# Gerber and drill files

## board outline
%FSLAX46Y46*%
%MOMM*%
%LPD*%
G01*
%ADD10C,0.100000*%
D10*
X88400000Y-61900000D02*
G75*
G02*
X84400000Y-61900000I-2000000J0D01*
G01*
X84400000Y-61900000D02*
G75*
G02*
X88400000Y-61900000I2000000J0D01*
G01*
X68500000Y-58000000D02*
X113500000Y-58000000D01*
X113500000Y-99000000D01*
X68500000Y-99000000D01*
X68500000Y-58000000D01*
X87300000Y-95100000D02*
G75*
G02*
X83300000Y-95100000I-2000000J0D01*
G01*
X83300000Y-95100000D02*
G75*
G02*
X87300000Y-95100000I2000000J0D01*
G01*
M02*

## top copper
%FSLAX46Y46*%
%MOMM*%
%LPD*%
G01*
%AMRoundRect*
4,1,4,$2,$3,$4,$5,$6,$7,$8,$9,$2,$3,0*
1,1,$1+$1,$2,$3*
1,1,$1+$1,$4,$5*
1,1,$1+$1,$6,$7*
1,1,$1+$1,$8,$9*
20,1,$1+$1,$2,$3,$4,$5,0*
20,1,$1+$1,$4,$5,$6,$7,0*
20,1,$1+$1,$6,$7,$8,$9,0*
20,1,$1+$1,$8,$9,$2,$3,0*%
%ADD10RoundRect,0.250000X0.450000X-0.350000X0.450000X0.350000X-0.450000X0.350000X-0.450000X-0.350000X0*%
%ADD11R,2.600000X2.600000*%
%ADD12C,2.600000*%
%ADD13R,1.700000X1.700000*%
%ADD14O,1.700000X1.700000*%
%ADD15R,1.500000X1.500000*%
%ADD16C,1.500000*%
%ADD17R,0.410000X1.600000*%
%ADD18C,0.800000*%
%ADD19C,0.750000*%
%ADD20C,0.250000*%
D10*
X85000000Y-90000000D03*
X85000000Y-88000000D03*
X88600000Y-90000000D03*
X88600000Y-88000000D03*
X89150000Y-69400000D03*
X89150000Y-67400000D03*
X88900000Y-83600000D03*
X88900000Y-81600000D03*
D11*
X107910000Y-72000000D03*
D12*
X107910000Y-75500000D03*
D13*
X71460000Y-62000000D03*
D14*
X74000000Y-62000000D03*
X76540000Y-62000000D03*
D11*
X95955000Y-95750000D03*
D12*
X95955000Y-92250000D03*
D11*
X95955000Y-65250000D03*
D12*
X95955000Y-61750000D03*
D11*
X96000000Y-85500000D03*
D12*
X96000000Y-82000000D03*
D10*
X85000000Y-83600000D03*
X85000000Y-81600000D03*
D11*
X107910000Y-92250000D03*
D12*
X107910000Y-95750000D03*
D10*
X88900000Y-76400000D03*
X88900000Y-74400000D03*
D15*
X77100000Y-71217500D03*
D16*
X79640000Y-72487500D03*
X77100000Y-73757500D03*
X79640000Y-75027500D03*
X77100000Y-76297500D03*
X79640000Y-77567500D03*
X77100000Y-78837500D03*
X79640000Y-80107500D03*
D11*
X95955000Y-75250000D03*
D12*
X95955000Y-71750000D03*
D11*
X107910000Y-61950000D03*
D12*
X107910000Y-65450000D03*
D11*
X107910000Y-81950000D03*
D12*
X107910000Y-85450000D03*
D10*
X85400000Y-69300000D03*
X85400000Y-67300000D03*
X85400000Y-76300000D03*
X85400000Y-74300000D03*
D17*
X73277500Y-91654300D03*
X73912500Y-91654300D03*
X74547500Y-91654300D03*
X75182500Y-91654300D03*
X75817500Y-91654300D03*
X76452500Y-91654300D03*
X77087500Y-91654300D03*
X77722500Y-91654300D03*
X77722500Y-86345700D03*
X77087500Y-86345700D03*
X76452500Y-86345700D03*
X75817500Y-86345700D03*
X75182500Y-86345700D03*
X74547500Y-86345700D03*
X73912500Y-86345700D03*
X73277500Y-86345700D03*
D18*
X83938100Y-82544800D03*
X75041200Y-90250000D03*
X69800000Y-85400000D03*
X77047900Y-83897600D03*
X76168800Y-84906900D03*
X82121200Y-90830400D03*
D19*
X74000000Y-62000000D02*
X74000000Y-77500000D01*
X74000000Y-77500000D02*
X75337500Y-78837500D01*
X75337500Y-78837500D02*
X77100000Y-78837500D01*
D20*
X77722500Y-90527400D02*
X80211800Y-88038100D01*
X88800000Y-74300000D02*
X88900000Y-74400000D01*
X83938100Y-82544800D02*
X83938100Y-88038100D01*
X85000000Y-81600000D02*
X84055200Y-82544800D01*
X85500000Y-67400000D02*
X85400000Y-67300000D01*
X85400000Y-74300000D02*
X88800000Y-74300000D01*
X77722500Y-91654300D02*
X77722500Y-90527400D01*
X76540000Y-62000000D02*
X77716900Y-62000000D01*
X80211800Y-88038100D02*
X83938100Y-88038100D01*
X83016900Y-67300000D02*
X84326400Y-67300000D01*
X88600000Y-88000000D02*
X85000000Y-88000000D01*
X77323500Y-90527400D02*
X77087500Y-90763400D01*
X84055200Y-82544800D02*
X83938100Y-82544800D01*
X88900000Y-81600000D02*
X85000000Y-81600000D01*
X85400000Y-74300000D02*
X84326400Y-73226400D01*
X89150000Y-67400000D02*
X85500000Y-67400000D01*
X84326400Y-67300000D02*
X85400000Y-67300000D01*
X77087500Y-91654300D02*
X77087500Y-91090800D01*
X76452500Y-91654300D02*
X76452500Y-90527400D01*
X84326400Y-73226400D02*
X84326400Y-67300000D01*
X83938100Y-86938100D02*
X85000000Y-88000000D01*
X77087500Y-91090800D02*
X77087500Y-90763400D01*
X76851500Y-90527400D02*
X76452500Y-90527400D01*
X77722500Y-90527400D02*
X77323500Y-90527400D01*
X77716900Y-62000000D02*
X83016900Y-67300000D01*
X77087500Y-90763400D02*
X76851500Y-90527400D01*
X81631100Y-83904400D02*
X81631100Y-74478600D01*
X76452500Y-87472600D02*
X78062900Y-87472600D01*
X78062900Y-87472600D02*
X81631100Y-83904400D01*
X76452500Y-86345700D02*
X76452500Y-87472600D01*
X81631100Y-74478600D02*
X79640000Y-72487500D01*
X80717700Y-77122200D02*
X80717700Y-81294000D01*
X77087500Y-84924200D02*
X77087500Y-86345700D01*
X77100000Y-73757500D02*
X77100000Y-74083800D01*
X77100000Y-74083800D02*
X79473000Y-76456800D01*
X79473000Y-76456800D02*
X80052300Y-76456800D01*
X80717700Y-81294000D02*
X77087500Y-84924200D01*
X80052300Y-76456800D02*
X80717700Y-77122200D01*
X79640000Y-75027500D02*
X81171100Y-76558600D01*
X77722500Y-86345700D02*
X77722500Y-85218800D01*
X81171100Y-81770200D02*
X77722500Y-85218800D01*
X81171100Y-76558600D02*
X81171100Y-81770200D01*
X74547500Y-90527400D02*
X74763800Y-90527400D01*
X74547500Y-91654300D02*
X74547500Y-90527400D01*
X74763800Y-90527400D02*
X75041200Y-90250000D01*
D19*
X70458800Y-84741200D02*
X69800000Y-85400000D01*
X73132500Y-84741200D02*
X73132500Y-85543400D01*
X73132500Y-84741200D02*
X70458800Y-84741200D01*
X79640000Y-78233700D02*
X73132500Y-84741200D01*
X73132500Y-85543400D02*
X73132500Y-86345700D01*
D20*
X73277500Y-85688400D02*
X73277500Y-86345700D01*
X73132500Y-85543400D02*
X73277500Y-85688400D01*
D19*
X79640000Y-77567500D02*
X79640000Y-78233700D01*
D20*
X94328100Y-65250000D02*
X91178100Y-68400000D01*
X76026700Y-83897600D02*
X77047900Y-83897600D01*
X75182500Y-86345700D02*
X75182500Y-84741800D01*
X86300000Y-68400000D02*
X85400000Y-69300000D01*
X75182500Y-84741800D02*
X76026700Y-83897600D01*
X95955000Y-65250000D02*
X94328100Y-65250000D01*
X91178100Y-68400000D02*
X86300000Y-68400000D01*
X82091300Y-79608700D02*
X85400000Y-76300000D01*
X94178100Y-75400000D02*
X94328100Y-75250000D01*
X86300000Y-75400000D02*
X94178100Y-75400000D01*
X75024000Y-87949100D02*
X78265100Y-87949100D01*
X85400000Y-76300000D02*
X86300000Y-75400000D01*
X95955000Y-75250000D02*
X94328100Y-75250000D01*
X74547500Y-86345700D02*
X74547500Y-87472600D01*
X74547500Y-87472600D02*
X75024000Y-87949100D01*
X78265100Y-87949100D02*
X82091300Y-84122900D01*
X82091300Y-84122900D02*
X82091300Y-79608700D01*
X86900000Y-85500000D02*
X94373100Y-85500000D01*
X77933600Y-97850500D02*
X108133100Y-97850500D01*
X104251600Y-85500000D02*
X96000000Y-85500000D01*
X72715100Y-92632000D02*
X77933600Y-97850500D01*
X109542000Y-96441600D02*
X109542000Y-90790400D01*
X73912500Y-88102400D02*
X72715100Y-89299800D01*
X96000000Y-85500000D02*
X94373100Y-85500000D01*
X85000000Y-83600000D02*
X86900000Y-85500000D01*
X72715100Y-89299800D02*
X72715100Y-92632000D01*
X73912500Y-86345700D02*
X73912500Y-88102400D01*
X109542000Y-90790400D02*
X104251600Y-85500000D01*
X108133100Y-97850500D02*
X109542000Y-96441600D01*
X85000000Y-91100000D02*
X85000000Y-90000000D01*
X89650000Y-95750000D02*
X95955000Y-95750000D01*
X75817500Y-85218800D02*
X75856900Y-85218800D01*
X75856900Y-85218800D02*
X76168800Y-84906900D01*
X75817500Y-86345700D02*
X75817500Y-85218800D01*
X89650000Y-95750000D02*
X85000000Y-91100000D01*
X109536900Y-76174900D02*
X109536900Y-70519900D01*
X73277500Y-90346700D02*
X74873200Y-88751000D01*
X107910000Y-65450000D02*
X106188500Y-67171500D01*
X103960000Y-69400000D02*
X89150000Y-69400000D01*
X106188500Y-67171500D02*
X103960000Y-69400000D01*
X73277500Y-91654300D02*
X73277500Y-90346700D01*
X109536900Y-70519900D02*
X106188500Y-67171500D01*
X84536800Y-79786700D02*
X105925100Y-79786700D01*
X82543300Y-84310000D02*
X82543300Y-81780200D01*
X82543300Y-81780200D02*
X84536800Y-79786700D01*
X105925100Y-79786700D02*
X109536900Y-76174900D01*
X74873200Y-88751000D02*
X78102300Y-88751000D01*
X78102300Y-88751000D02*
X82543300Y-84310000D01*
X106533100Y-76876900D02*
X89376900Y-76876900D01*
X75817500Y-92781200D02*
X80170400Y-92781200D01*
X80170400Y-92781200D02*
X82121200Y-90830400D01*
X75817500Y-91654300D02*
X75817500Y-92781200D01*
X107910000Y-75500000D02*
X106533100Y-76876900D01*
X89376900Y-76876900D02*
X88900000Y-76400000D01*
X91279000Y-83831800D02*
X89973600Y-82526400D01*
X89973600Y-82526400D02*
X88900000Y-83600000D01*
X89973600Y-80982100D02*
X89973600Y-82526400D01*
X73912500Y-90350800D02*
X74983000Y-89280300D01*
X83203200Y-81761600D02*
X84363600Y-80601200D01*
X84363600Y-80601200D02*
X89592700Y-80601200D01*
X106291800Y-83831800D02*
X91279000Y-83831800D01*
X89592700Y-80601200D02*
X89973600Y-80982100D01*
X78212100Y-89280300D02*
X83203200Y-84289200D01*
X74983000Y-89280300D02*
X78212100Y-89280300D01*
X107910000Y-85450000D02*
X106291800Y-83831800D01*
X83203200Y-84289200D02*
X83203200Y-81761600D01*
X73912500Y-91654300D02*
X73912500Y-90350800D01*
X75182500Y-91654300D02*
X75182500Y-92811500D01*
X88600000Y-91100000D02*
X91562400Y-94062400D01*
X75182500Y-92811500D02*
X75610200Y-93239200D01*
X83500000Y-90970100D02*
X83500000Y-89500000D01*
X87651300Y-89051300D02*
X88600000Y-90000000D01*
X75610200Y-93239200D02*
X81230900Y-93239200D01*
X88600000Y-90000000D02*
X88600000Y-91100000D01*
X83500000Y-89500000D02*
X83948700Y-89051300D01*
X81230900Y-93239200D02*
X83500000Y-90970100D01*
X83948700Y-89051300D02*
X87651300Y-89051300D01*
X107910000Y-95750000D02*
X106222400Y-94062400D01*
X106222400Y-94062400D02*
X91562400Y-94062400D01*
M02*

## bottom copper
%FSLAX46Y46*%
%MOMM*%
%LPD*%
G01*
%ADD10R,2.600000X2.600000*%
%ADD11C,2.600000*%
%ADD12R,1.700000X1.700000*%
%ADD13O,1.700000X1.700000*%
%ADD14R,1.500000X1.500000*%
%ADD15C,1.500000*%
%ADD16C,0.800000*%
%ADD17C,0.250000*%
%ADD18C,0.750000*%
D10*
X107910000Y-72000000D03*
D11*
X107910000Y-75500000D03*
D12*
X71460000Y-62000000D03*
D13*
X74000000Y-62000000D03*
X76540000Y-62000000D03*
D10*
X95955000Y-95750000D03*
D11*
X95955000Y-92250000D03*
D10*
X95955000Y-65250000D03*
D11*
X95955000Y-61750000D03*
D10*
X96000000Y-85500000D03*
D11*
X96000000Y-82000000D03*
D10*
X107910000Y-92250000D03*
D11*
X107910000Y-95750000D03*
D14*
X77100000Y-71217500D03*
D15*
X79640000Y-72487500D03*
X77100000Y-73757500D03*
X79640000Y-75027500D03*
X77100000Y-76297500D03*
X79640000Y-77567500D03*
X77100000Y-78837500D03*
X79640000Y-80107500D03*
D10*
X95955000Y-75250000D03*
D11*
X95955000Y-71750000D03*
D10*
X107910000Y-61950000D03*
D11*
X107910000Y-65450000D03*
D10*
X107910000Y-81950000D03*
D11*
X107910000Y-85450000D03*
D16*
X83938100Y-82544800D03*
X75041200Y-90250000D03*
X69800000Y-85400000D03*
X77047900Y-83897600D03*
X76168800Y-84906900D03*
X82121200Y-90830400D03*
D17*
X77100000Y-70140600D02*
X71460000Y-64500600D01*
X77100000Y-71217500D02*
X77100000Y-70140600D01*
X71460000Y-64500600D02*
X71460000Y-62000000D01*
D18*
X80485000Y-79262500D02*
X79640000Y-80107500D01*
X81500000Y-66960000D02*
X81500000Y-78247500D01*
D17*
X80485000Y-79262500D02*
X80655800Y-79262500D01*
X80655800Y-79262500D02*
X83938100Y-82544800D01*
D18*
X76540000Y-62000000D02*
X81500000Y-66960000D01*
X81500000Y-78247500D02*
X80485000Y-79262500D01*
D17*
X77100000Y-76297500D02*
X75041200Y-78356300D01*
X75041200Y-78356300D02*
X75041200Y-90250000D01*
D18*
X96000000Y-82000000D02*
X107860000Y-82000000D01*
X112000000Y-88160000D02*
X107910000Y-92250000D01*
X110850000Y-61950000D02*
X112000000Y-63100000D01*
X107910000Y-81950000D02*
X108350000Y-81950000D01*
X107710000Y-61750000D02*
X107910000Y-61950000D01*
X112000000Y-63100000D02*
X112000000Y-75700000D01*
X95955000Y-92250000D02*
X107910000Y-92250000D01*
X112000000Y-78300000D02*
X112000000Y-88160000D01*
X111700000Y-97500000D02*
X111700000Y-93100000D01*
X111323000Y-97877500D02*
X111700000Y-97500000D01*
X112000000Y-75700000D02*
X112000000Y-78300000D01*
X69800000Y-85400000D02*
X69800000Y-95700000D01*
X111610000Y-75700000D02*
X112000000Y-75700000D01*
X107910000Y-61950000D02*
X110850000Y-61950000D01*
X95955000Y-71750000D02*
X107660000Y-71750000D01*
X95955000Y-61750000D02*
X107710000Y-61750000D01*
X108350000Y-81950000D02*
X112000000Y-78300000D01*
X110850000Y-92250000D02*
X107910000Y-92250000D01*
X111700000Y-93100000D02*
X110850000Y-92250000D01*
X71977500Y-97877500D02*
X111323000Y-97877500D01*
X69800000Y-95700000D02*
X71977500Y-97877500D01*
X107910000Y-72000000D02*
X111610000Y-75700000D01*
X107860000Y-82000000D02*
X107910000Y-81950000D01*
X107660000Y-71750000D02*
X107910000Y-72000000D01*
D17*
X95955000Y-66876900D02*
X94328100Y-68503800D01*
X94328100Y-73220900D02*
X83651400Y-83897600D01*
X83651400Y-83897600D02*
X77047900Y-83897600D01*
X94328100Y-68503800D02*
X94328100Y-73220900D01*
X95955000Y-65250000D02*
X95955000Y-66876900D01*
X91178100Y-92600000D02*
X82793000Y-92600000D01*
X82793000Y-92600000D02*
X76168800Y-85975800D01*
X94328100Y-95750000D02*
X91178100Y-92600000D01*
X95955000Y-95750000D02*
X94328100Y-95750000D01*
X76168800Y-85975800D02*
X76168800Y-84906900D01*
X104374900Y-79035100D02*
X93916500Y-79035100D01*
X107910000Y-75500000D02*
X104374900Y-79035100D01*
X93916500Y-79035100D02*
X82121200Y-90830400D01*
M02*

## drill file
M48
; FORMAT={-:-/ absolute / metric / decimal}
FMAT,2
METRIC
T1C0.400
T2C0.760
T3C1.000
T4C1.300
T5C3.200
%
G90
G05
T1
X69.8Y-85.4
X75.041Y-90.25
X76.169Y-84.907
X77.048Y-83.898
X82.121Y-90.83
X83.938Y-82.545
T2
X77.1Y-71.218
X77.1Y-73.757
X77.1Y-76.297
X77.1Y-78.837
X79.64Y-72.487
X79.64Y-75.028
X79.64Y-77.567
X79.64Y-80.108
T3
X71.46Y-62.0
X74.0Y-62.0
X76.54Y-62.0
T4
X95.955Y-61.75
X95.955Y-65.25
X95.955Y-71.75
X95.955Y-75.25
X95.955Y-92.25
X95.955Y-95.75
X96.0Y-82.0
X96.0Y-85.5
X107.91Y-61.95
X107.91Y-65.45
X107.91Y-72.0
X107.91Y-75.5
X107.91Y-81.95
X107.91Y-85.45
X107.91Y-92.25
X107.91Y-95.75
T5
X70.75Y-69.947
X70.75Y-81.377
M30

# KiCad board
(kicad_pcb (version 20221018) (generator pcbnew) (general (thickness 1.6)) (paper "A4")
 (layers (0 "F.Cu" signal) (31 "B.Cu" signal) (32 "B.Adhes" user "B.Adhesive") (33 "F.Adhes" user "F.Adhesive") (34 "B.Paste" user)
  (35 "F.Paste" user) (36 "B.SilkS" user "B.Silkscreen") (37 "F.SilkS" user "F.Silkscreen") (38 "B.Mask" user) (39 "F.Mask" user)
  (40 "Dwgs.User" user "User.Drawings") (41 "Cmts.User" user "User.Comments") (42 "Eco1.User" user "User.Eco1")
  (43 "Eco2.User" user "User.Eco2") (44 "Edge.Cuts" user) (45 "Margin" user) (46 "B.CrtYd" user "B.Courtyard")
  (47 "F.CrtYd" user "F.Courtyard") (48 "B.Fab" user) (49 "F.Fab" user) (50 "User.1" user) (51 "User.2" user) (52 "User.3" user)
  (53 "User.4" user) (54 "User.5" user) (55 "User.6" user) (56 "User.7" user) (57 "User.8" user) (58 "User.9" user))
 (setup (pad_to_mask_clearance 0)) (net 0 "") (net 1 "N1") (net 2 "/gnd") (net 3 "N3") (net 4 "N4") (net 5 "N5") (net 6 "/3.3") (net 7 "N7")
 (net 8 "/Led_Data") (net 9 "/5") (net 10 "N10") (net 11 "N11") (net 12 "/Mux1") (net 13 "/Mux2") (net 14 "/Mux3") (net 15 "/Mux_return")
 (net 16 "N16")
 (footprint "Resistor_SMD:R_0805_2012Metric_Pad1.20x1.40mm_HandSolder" (layer "F.Cu") (at 85 89 90)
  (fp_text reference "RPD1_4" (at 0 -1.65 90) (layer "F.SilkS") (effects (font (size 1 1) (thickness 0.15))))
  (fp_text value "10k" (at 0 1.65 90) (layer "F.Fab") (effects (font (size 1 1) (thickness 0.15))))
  (pad "1" smd roundrect (at -1 0 90) (size 1.2 1.4) (layers "F.Cu" "F.Paste" "F.Mask") (roundrect_rratio 0.2083333333) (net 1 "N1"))
  (pad "2" smd roundrect (at 1 0 90) (size 1.2 1.4) (layers "F.Cu" "F.Paste" "F.Mask") (roundrect_rratio 0.2083333333) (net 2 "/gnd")))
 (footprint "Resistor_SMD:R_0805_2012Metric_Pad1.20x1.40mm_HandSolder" (layer "F.Cu") (at 88.6 89 90)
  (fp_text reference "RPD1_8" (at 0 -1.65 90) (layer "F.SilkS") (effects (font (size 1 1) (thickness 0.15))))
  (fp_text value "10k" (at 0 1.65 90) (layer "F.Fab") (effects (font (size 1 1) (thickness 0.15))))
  (pad "1" smd roundrect (at -1 0 90) (size 1.2 1.4) (layers "F.Cu" "F.Paste" "F.Mask") (roundrect_rratio 0.2083333333) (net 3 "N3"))
  (pad "2" smd roundrect (at 1 0 90) (size 1.2 1.4) (layers "F.Cu" "F.Paste" "F.Mask") (roundrect_rratio 0.2083333333) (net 2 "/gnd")))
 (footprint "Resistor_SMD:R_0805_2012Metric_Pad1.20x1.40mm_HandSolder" (layer "F.Cu") (at 89.15 68.4 90)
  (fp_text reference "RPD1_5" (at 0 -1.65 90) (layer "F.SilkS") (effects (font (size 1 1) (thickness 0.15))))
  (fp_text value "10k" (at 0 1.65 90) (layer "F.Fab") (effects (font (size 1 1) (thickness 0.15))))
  (pad "1" smd roundrect (at -1 0 90) (size 1.2 1.4) (layers "F.Cu" "F.Paste" "F.Mask") (roundrect_rratio 0.2083333333) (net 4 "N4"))
  (pad "2" smd roundrect (at 1 0 90) (size 1.2 1.4) (layers "F.Cu" "F.Paste" "F.Mask") (roundrect_rratio 0.2083333333) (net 2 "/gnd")))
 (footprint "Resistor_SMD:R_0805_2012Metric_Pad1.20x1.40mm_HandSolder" (layer "F.Cu") (at 88.9 82.6 90)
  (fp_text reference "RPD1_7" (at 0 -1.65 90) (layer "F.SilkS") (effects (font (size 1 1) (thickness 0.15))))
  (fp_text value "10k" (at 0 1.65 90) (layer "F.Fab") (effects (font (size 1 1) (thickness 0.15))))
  (pad "1" smd roundrect (at -1 0 90) (size 1.2 1.4) (layers "F.Cu" "F.Paste" "F.Mask") (roundrect_rratio 0.2083333333) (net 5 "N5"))
  (pad "2" smd roundrect (at 1 0 90) (size 1.2 1.4) (layers "F.Cu" "F.Paste" "F.Mask") (roundrect_rratio 0.2083333333) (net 2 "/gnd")))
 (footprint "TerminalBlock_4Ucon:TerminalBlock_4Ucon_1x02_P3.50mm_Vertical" (layer "F.Cu") (at 107.91 72 -90)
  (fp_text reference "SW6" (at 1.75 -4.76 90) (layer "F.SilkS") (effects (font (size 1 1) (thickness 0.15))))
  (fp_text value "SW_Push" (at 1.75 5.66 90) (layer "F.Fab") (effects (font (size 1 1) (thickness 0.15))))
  (pad "1" thru_hole rect (at 0 0 270) (size 2.6 2.6) (drill 1.3) (layers "*.Cu" "*.Mask") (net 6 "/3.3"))
  (pad "2" thru_hole circle (at 3.5 0 270) (size 2.6 2.6) (drill 1.3) (layers "*.Cu" "*.Mask") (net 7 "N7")))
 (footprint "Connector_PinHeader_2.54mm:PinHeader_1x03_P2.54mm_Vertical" (layer "F.Cu") (at 71.46 62 90)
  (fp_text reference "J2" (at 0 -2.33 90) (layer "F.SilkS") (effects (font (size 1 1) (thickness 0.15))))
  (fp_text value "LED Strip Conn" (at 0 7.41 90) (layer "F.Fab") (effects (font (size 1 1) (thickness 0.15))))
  (pad "1" thru_hole rect (at 0 0 90) (size 1.7 1.7) (drill 1) (layers "*.Cu" "*.Mask") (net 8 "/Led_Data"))
  (pad "2" thru_hole oval (at 0 2.54 90) (size 1.7 1.7) (drill 1) (layers "*.Cu" "*.Mask") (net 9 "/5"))
  (pad "3" thru_hole oval (at 0 5.08 90) (size 1.7 1.7) (drill 1) (layers "*.Cu" "*.Mask") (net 2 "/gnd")))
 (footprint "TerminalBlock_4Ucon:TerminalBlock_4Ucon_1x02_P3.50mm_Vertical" (layer "F.Cu") (at 95.955 95.75 90)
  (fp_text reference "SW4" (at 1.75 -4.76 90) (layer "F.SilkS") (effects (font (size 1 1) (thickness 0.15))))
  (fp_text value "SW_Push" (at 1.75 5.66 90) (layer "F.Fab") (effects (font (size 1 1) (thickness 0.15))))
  (pad "1" thru_hole rect (at 0 0 90) (size 2.6 2.6) (drill 1.3) (layers "*.Cu" "*.Mask") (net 1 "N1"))
  (pad "2" thru_hole circle (at 3.5 0 90) (size 2.6 2.6) (drill 1.3) (layers "*.Cu" "*.Mask") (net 6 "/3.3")))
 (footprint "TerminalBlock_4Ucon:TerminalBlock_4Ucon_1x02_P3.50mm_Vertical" (layer "F.Cu") (at 95.955 65.25 90)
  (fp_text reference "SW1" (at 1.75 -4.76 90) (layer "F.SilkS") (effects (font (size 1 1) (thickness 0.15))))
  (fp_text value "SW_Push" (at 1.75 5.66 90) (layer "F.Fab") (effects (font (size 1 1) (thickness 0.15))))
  (pad "1" thru_hole rect (at 0 0 90) (size 2.6 2.6) (drill 1.3) (layers "*.Cu" "*.Mask") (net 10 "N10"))
  (pad "2" thru_hole circle (at 3.5 0 90) (size 2.6 2.6) (drill 1.3) (layers "*.Cu" "*.Mask") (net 6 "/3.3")))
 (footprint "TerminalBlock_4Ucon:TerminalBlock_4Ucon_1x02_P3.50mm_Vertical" (layer "F.Cu") (at 96 85.5 90)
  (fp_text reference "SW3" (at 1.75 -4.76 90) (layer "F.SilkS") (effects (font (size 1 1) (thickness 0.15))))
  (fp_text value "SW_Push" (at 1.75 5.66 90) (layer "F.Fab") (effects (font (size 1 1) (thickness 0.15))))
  (pad "1" thru_hole rect (at 0 0 90) (size 2.6 2.6) (drill 1.3) (layers "*.Cu" "*.Mask") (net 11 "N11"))
  (pad "2" thru_hole circle (at 3.5 0 90) (size 2.6 2.6) (drill 1.3) (layers "*.Cu" "*.Mask") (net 6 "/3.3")))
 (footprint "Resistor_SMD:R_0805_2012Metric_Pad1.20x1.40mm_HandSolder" (layer "F.Cu") (at 85 82.6 90)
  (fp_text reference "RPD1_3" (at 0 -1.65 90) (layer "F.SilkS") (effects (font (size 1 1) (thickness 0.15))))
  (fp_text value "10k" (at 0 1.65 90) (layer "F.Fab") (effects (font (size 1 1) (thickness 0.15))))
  (pad "1" smd roundrect (at -1 0 90) (size 1.2 1.4) (layers "F.Cu" "F.Paste" "F.Mask") (roundrect_rratio 0.2083333333) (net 11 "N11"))
  (pad "2" smd roundrect (at 1 0 90) (size 1.2 1.4) (layers "F.Cu" "F.Paste" "F.Mask") (roundrect_rratio 0.2083333333) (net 2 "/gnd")))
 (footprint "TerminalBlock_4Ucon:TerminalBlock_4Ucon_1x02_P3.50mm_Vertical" (layer "F.Cu") (at 107.91 92.25 -90)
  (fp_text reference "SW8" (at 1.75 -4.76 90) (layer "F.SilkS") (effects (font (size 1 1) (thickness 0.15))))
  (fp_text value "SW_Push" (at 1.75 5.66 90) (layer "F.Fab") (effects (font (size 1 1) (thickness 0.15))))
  (pad "1" thru_hole rect (at 0 0 270) (size 2.6 2.6) (drill 1.3) (layers "*.Cu" "*.Mask") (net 6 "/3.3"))
  (pad "2" thru_hole circle (at 3.5 0 270) (size 2.6 2.6) (drill 1.3) (layers "*.Cu" "*.Mask") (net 3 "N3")))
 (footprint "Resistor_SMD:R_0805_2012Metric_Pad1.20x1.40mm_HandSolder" (layer "F.Cu") (at 88.9 75.4 90)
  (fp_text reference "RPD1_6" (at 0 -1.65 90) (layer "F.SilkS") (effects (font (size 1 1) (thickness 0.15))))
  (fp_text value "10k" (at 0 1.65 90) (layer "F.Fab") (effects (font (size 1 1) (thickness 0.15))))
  (pad "1" smd roundrect (at -1 0 90) (size 1.2 1.4) (layers "F.Cu" "F.Paste" "F.Mask") (roundrect_rratio 0.2083333333) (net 7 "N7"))
  (pad "2" smd roundrect (at 1 0 90) (size 1.2 1.4) (layers "F.Cu" "F.Paste" "F.Mask") (roundrect_rratio 0.2083333333) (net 2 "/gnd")))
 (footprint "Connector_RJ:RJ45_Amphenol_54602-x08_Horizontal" (layer "F.Cu") (at 77.1 71.2175 -90)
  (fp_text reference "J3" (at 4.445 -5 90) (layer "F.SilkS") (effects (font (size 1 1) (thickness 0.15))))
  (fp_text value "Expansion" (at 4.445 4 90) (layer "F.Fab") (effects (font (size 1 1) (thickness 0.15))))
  (pad "" np_thru_hole circle (at -1.27 6.35 270) (size 3.2 3.2) (drill 3.2) (layers "*.Cu" "*.Mask"))
  (pad "" np_thru_hole circle (at 10.16 6.35 270) (size 3.2 3.2) (drill 3.2) (layers "*.Cu" "*.Mask"))
  (pad "1" thru_hole rect (at 0 0 270) (size 1.5 1.5) (drill 0.76) (layers "*.Cu" "*.Mask") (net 8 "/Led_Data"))
  (pad "2" thru_hole circle (at 1.27 -2.54 270) (size 1.5 1.5) (drill 0.76) (layers "*.Cu" "*.Mask") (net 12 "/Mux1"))
  (pad "3" thru_hole circle (at 2.54 0 270) (size 1.5 1.5) (drill 0.76) (layers "*.Cu" "*.Mask") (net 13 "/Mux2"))
  (pad "4" thru_hole circle (at 3.81 -2.54 270) (size 1.5 1.5) (drill 0.76) (layers "*.Cu" "*.Mask") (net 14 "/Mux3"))
  (pad "5" thru_hole circle (at 5.08 0 270) (size 1.5 1.5) (drill 0.76) (layers "*.Cu" "*.Mask") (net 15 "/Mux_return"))
  (pad "6" thru_hole circle (at 6.35 -2.54 270) (size 1.5 1.5) (drill 0.76) (layers "*.Cu" "*.Mask") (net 6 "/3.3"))
  (pad "7" thru_hole circle (at 7.62 0 270) (size 1.5 1.5) (drill 0.76) (layers "*.Cu" "*.Mask") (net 9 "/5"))
  (pad "8" thru_hole circle (at 8.89 -2.54 270) (size 1.5 1.5) (drill 0.76) (layers "*.Cu" "*.Mask") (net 2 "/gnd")))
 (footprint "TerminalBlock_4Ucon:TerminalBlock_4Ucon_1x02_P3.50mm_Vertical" (layer "F.Cu") (at 95.955 75.25 90)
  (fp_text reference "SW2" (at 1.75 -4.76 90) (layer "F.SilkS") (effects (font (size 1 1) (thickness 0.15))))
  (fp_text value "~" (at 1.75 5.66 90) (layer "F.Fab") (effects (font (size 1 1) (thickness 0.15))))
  (pad "1" thru_hole rect (at 0 0 90) (size 2.6 2.6) (drill 1.3) (layers "*.Cu" "*.Mask") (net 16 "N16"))
  (pad "2" thru_hole circle (at 3.5 0 90) (size 2.6 2.6) (drill 1.3) (layers "*.Cu" "*.Mask") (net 6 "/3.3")))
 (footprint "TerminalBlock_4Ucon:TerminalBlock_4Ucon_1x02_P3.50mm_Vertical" (layer "F.Cu") (at 107.91 61.95 -90)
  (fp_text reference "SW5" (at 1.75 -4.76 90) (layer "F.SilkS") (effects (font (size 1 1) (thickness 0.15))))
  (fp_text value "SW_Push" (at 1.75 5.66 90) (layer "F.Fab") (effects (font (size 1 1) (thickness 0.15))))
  (pad "1" thru_hole rect (at 0 0 270) (size 2.6 2.6) (drill 1.3) (layers "*.Cu" "*.Mask") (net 6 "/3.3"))
  (pad "2" thru_hole circle (at 3.5 0 270) (size 2.6 2.6) (drill 1.3) (layers "*.Cu" "*.Mask") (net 4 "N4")))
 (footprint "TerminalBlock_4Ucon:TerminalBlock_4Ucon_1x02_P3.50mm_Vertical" (layer "F.Cu") (at 107.91 81.95 -90)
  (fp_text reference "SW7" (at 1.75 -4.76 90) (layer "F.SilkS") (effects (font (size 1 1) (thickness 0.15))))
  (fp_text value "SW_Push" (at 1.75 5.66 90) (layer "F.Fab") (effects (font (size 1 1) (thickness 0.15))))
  (pad "1" thru_hole rect (at 0 0 270) (size 2.6 2.6) (drill 1.3) (layers "*.Cu" "*.Mask") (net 6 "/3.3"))
  (pad "2" thru_hole circle (at 3.5 0 270) (size 2.6 2.6) (drill 1.3) (layers "*.Cu" "*.Mask") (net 5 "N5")))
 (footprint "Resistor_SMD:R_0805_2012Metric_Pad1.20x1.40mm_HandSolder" (layer "F.Cu") (at 85.4 68.3 90)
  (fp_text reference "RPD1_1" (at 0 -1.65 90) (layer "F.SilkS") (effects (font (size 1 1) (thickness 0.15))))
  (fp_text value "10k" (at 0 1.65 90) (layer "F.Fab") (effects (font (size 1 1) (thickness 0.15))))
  (pad "1" smd roundrect (at -1 0 90) (size 1.2 1.4) (layers "F.Cu" "F.Paste" "F.Mask") (roundrect_rratio 0.2083333333) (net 10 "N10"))
  (pad "2" smd roundrect (at 1 0 90) (size 1.2 1.4) (layers "F.Cu" "F.Paste" "F.Mask") (roundrect_rratio 0.2083333333) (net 2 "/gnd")))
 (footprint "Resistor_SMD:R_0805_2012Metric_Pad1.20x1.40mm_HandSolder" (layer "F.Cu") (at 85.4 75.3 90)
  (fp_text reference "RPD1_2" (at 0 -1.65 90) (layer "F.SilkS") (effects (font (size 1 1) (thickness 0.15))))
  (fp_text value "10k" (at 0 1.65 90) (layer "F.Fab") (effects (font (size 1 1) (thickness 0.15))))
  (pad "1" smd roundrect (at -1 0 90) (size 1.2 1.4) (layers "F.Cu" "F.Paste" "F.Mask") (roundrect_rratio 0.2083333333) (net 16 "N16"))
  (pad "2" smd roundrect (at 1 0 90) (size 1.2 1.4) (layers "F.Cu" "F.Paste" "F.Mask") (roundrect_rratio 0.2083333333) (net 2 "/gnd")))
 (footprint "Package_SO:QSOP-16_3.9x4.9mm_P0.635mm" (layer "F.Cu") (at 75.5 89 90)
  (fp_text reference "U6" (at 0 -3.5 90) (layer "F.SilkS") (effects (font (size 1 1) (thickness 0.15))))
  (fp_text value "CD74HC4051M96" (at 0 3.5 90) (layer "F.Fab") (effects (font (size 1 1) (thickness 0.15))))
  (pad "1" smd rect (at -2.6543 -2.2225 90) (size 1.6 0.41) (layers "F.Cu" "F.Paste" "F.Mask") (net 4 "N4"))
  (pad "2" smd rect (at -2.6543 -1.5875 90) (size 1.6 0.41) (layers "F.Cu" "F.Paste" "F.Mask") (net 5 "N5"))
  (pad "3" smd rect (at -2.6543 -0.9525 90) (size 1.6 0.41) (layers "F.Cu" "F.Paste" "F.Mask") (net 15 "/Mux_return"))
  (pad "4" smd rect (at -2.6543 -0.3175 90) (size 1.6 0.41) (layers "F.Cu" "F.Paste" "F.Mask") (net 3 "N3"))
  (pad "5" smd rect (at -2.6543 0.3175 90) (size 1.6 0.41) (layers "F.Cu" "F.Paste" "F.Mask") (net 7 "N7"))
  (pad "6" smd rect (at -2.6543 0.9525 90) (size 1.6 0.41) (layers "F.Cu" "F.Paste" "F.Mask") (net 2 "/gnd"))
  (pad "7" smd rect (at -2.6543 1.5875 90) (size 1.6 0.41) (layers "F.Cu" "F.Paste" "F.Mask") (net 2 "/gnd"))
  (pad "8" smd rect (at -2.6543 2.2225 90) (size 1.6 0.41) (layers "F.Cu" "F.Paste" "F.Mask") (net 2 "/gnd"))
  (pad "9" smd rect (at 2.6543 2.2225 90) (size 1.6 0.41) (layers "F.Cu" "F.Paste" "F.Mask") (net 14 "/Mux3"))
  (pad "10" smd rect (at 2.6543 1.5875 90) (size 1.6 0.41) (layers "F.Cu" "F.Paste" "F.Mask") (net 13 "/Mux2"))
  (pad "11" smd rect (at 2.6543 0.9525 90) (size 1.6 0.41) (layers "F.Cu" "F.Paste" "F.Mask") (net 12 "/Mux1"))
  (pad "12" smd rect (at 2.6543 0.3175 90) (size 1.6 0.41) (layers "F.Cu" "F.Paste" "F.Mask") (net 1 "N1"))
  (pad "13" smd rect (at 2.6543 -0.3175 90) (size 1.6 0.41) (layers "F.Cu" "F.Paste" "F.Mask") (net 10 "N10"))
  (pad "14" smd rect (at 2.6543 -0.9525 90) (size 1.6 0.41) (layers "F.Cu" "F.Paste" "F.Mask") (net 16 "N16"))
  (pad "15" smd rect (at 2.6543 -1.5875 90) (size 1.6 0.41) (layers "F.Cu" "F.Paste" "F.Mask") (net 11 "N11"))
  (pad "16" smd rect (at 2.6543 -2.2225 90) (size 1.6 0.41) (layers "F.Cu" "F.Paste" "F.Mask") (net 6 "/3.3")))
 (gr_circle (center 86.4 61.9) (end 88.4 61.9) (stroke (width 0.1) (type default)) (fill none) (layer "Edge.Cuts"))
 (gr_rect (start 68.5 58) (end 113.5 99) (stroke (width 0.1) (type default)) (fill none) (layer "Edge.Cuts"))
 (gr_circle (center 85.3 95.1) (end 87.3 95.1) (stroke (width 0.1) (type default)) (fill none) (layer "Edge.Cuts"))
 (segment (start 77.1 70.1406) (end 71.46 64.5006) (width 0.25) (layer "B.Cu") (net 8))
 (segment (start 77.1 71.2175) (end 77.1 70.1406) (width 0.25) (layer "B.Cu") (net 8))
 (segment (start 71.46 64.5006) (end 71.46 62) (width 0.25) (layer "B.Cu") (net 8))
 (segment (start 74 62) (end 74 77.5) (width 0.75) (layer "F.Cu") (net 9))
 (segment (start 74 77.5) (end 75.3375 78.8375) (width 0.75) (layer "F.Cu") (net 9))
 (segment (start 75.3375 78.8375) (end 77.1 78.8375) (width 0.75) (layer "F.Cu") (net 9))
 (segment (start 77.7225 90.5274) (end 80.2118 88.0381) (width 0.25) (layer "F.Cu") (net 2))
 (segment (start 88.8 74.3) (end 88.9 74.4) (width 0.25) (layer "F.Cu") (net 2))
 (segment (start 83.9381 82.5448) (end 83.9381 88.0381) (width 0.25) (layer "F.Cu") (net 2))
 (segment (start 85 81.6) (end 84.0552 82.5448) (width 0.25) (layer "F.Cu") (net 2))
 (segment (start 85.5 67.4) (end 85.4 67.3) (width 0.25) (layer "F.Cu") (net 2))
 (segment (start 85.4 74.3) (end 88.8 74.3) (width 0.25) (layer "F.Cu") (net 2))
 (segment (start 77.7225 91.6543) (end 77.7225 90.5274) (width 0.25) (layer "F.Cu") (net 2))
 (segment (start 76.54 62) (end 77.7169 62) (width 0.25) (layer "F.Cu") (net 2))
 (segment (start 80.2118 88.0381) (end 83.9381 88.0381) (width 0.25) (layer "F.Cu") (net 2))
 (segment (start 83.0169 67.3) (end 84.3264 67.3) (width 0.25) (layer "F.Cu") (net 2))
 (segment (start 88.6 88) (end 85 88) (width 0.25) (layer "F.Cu") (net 2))
 (segment (start 77.3235 90.5274) (end 77.0875 90.7634) (width 0.25) (layer "F.Cu") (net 2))
 (segment (start 84.0552 82.5448) (end 83.9381 82.5448) (width 0.25) (layer "F.Cu") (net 2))
 (segment (start 88.9 81.6) (end 85 81.6) (width 0.25) (layer "F.Cu") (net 2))
 (segment (start 85.4 74.3) (end 84.3264 73.2264) (width 0.25) (layer "F.Cu") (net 2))
 (segment (start 89.15 67.4) (end 85.5 67.4) (width 0.25) (layer "F.Cu") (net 2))
 (segment (start 84.3264 67.3) (end 85.4 67.3) (width 0.25) (layer "F.Cu") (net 2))
 (segment (start 77.0875 91.6543) (end 77.0875 91.0908) (width 0.25) (layer "F.Cu") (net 2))
 (segment (start 76.4525 91.6543) (end 76.4525 90.5274) (width 0.25) (layer "F.Cu") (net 2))
 (segment (start 84.3264 73.2264) (end 84.3264 67.3) (width 0.25) (layer "F.Cu") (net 2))
 (segment (start 83.9381 86.9381) (end 85 88) (width 0.25) (layer "F.Cu") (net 2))
 (segment (start 77.0875 91.0908) (end 77.0875 90.7634) (width 0.25) (layer "F.Cu") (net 2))
 (segment (start 76.8515 90.5274) (end 76.4525 90.5274) (width 0.25) (layer "F.Cu") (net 2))
 (segment (start 77.7225 90.5274) (end 77.3235 90.5274) (width 0.25) (layer "F.Cu") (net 2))
 (segment (start 77.7169 62) (end 83.0169 67.3) (width 0.25) (layer "F.Cu") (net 2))
 (segment (start 77.0875 90.7634) (end 76.8515 90.5274) (width 0.25) (layer "F.Cu") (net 2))
 (via (at 83.9381 82.5448) (size 0.8) (drill 0.4) (layers "F.Cu" "B.Cu") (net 2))
 (segment (start 80.485 79.2625) (end 79.64 80.1075) (width 0.75) (layer "B.Cu") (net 2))
 (segment (start 81.5 66.96) (end 81.5 78.2475) (width 0.75) (layer "B.Cu") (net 2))
 (segment (start 80.485 79.2625) (end 80.6558 79.2625) (width 0.25) (layer "B.Cu") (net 2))
 (segment (start 80.6558 79.2625) (end 83.9381 82.5448) (width 0.25) (layer "B.Cu") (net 2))
 (segment (start 76.54 62) (end 81.5 66.96) (width 0.75) (layer "B.Cu") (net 2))
 (segment (start 81.5 78.2475) (end 80.485 79.2625) (width 0.75) (layer "B.Cu") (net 2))
 (segment (start 81.6311 83.9044) (end 81.6311 74.4786) (width 0.25) (layer "F.Cu") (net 12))
 (segment (start 76.4525 87.4726) (end 78.0629 87.4726) (width 0.25) (layer "F.Cu") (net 12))
 (segment (start 78.0629 87.4726) (end 81.6311 83.9044) (width 0.25) (layer "F.Cu") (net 12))
 (segment (start 76.4525 86.3457) (end 76.4525 87.4726) (width 0.25) (layer "F.Cu") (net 12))
 (segment (start 81.6311 74.4786) (end 79.64 72.4875) (width 0.25) (layer "F.Cu") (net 12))
 (segment (start 80.7177 77.1222) (end 80.7177 81.294) (width 0.25) (layer "F.Cu") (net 13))
 (segment (start 77.0875 84.9242) (end 77.0875 86.3457) (width 0.25) (layer "F.Cu") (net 13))
 (segment (start 77.1 73.7575) (end 77.1 74.0838) (width 0.25) (layer "F.Cu") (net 13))
 (segment (start 77.1 74.0838) (end 79.473 76.4568) (width 0.25) (layer "F.Cu") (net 13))
 (segment (start 79.473 76.4568) (end 80.0523 76.4568) (width 0.25) (layer "F.Cu") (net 13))
 (segment (start 80.7177 81.294) (end 77.0875 84.9242) (width 0.25) (layer "F.Cu") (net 13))
 (segment (start 80.0523 76.4568) (end 80.7177 77.1222) (width 0.25) (layer "F.Cu") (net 13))
 (segment (start 79.64 75.0275) (end 81.1711 76.5586) (width 0.25) (layer "F.Cu") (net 14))
 (segment (start 77.7225 86.3457) (end 77.7225 85.2188) (width 0.25) (layer "F.Cu") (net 14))
 (segment (start 81.1711 81.7702) (end 77.7225 85.2188) (width 0.25) (layer "F.Cu") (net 14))
 (segment (start 81.1711 76.5586) (end 81.1711 81.7702) (width 0.25) (layer "F.Cu") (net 14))
 (segment (start 74.5475 90.5274) (end 74.7638 90.5274) (width 0.25) (layer "F.Cu") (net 15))
 (segment (start 74.5475 91.6543) (end 74.5475 90.5274) (width 0.25) (layer "F.Cu") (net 15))
 (segment (start 74.7638 90.5274) (end 75.0412 90.25) (width 0.25) (layer "F.Cu") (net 15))
 (via (at 75.0412 90.25) (size 0.8) (drill 0.4) (layers "F.Cu" "B.Cu") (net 15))
 (segment (start 77.1 76.2975) (end 75.0412 78.3563) (width 0.25) (layer "B.Cu") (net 15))
 (segment (start 75.0412 78.3563) (end 75.0412 90.25) (width 0.25) (layer "B.Cu") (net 15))
 (segment (start 70.4588 84.7412) (end 69.8 85.4) (width 0.75) (layer "F.Cu") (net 6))
 (segment (start 73.1325 84.7412) (end 73.1325 85.5434) (width 0.75) (layer "F.Cu") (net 6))
 (segment (start 73.1325 84.7412) (end 70.4588 84.7412) (width 0.75) (layer "F.Cu") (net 6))
 (segment (start 79.64 78.2337) (end 73.1325 84.7412) (width 0.75) (layer "F.Cu") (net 6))
 (segment (start 73.1325 85.5434) (end 73.1325 86.3457) (width 0.75) (layer "F.Cu") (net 6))
 (segment (start 73.2775 85.6884) (end 73.2775 86.3457) (width 0.25) (layer "F.Cu") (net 6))
 (segment (start 73.1325 85.5434) (end 73.2775 85.6884) (width 0.25) (layer "F.Cu") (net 6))
 (segment (start 79.64 77.5675) (end 79.64 78.2337) (width 0.75) (layer "F.Cu") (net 6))
 (via (at 69.8 85.4) (size 0.8) (drill 0.4) (layers "F.Cu" "B.Cu") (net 6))
 (segment (start 96 82) (end 107.86 82) (width 0.75) (layer "B.Cu") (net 6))
 (segment (start 112 88.16) (end 107.91 92.25) (width 0.75) (layer "B.Cu") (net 6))
 (segment (start 110.85 61.95) (end 112 63.1) (width 0.75) (layer "B.Cu") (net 6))
 (segment (start 107.91 81.95) (end 108.35 81.95) (width 0.75) (layer "B.Cu") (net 6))
 (segment (start 107.71 61.75) (end 107.91 61.95) (width 0.75) (layer "B.Cu") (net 6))
 (segment (start 112 63.1) (end 112 75.7) (width 0.75) (layer "B.Cu") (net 6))
 (segment (start 95.955 92.25) (end 107.91 92.25) (width 0.75) (layer "B.Cu") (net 6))
 (segment (start 112 78.3) (end 112 88.16) (width 0.75) (layer "B.Cu") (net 6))
 (segment (start 111.7 97.5) (end 111.7 93.1) (width 0.75) (layer "B.Cu") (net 6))
 (segment (start 111.323 97.8775) (end 111.7 97.5) (width 0.75) (layer "B.Cu") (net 6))
 (segment (start 112 75.7) (end 112 78.3) (width 0.75) (layer "B.Cu") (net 6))
 (segment (start 69.8 85.4) (end 69.8 95.7) (width 0.75) (layer "B.Cu") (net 6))
 (segment (start 111.61 75.7) (end 112 75.7) (width 0.75) (layer "B.Cu") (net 6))
 (segment (start 107.91 61.95) (end 110.85 61.95) (width 0.75) (layer "B.Cu") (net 6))
 (segment (start 95.955 71.75) (end 107.66 71.75) (width 0.75) (layer "B.Cu") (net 6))
 (segment (start 95.955 61.75) (end 107.71 61.75) (width 0.75) (layer "B.Cu") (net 6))
 (segment (start 108.35 81.95) (end 112 78.3) (width 0.75) (layer "B.Cu") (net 6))
 (segment (start 110.85 92.25) (end 107.91 92.25) (width 0.75) (layer "B.Cu") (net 6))
 (segment (start 111.7 93.1) (end 110.85 92.25) (width 0.75) (layer "B.Cu") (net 6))
 (segment (start 71.9775 97.8775) (end 111.323 97.8775) (width 0.75) (layer "B.Cu") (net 6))
 (segment (start 69.8 95.7) (end 71.9775 97.8775) (width 0.75) (layer "B.Cu") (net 6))
 (segment (start 107.91 72) (end 111.61 75.7) (width 0.75) (layer "B.Cu") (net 6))
 (segment (start 107.86 82) (end 107.91 81.95) (width 0.75) (layer "B.Cu") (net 6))
 (segment (start 107.66 71.75) (end 107.91 72) (width 0.75) (layer "B.Cu") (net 6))
 (segment (start 94.3281 65.25) (end 91.1781 68.4) (width 0.25) (layer "F.Cu") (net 10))
 (segment (start 76.0267 83.8976) (end 77.0479 83.8976) (width 0.25) (layer "F.Cu") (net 10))
 (segment (start 75.1825 86.3457) (end 75.1825 84.7418) (width 0.25) (layer "F.Cu") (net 10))
 (segment (start 86.3 68.4) (end 85.4 69.3) (width 0.25) (layer "F.Cu") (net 10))
 (segment (start 75.1825 84.7418) (end 76.0267 83.8976) (width 0.25) (layer "F.Cu") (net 10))
 (segment (start 95.955 65.25) (end 94.3281 65.25) (width 0.25) (layer "F.Cu") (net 10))
 (segment (start 91.1781 68.4) (end 86.3 68.4) (width 0.25) (layer "F.Cu") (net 10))
 (via (at 77.0479 83.8976) (size 0.8) (drill 0.4) (layers "F.Cu" "B.Cu") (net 10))
 (segment (start 95.955 66.8769) (end 94.3281 68.5038) (width 0.25) (layer "B.Cu") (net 10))
 (segment (start 94.3281 73.2209) (end 83.6514 83.8976) (width 0.25) (layer "B.Cu") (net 10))
 (segment (start 83.6514 83.8976) (end 77.0479 83.8976) (width 0.25) (layer "B.Cu") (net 10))
 (segment (start 94.3281 68.5038) (end 94.3281 73.2209) (width 0.25) (layer "B.Cu") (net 10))
 (segment (start 95.955 65.25) (end 95.955 66.8769) (width 0.25) (layer "B.Cu") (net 10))
 (segment (start 82.0913 79.6087) (end 85.4 76.3) (width 0.25) (layer "F.Cu") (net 16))
 (segment (start 94.1781 75.4) (end 94.3281 75.25) (width 0.25) (layer "F.Cu") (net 16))
 (segment (start 86.3 75.4) (end 94.1781 75.4) (width 0.25) (layer "F.Cu") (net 16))
 (segment (start 75.024 87.9491) (end 78.2651 87.9491) (width 0.25) (layer "F.Cu") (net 16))
 (segment (start 85.4 76.3) (end 86.3 75.4) (width 0.25) (layer "F.Cu") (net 16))
 (segment (start 95.955 75.25) (end 94.3281 75.25) (width 0.25) (layer "F.Cu") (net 16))
 (segment (start 74.5475 86.3457) (end 74.5475 87.4726) (width 0.25) (layer "F.Cu") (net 16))
 (segment (start 74.5475 87.4726) (end 75.024 87.9491) (width 0.25) (layer "F.Cu") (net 16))
 (segment (start 78.2651 87.9491) (end 82.0913 84.1229) (width 0.25) (layer "F.Cu") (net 16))
 (segment (start 82.0913 84.1229) (end 82.0913 79.6087) (width 0.25) (layer "F.Cu") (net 16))
 (segment (start 86.9 85.5) (end 94.3731 85.5) (width 0.25) (layer "F.Cu") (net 11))
 (segment (start 77.9336 97.8505) (end 108.1331 97.8505) (width 0.25) (layer "F.Cu") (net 11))
 (segment (start 104.2516 85.5) (end 96 85.5) (width 0.25) (layer "F.Cu") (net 11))
 (segment (start 72.7151 92.632) (end 77.9336 97.8505) (width 0.25) (layer "F.Cu") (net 11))
 (segment (start 109.542 96.4416) (end 109.542 90.7904) (width 0.25) (layer "F.Cu") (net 11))
 (segment (start 73.9125 88.1024) (end 72.7151 89.2998) (width 0.25) (layer "F.Cu") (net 11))
 (segment (start 96 85.5) (end 94.3731 85.5) (width 0.25) (layer "F.Cu") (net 11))
 (segment (start 85 83.6) (end 86.9 85.5) (width 0.25) (layer "F.Cu") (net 11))
 (segment (start 72.7151 89.2998) (end 72.7151 92.632) (width 0.25) (layer "F.Cu") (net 11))
 (segment (start 73.9125 86.3457) (end 73.9125 88.1024) (width 0.25) (layer "F.Cu") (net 11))
 (segment (start 109.542 90.7904) (end 104.2516 85.5) (width 0.25) (layer "F.Cu") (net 11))
 (segment (start 108.1331 97.8505) (end 109.542 96.4416) (width 0.25) (layer "F.Cu") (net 11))
 (segment (start 85 91.1) (end 85 90) (width 0.25) (layer "F.Cu") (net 1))
 (segment (start 89.65 95.75) (end 95.955 95.75) (width 0.25) (layer "F.Cu") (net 1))
 (segment (start 75.8175 85.2188) (end 75.8569 85.2188) (width 0.25) (layer "F.Cu") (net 1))
 (segment (start 75.8569 85.2188) (end 76.1688 84.9069) (width 0.25) (layer "F.Cu") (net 1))
 (segment (start 75.8175 86.3457) (end 75.8175 85.2188) (width 0.25) (layer "F.Cu") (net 1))
 (segment (start 89.65 95.75) (end 85 91.1) (width 0.25) (layer "F.Cu") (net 1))
 (via (at 76.1688 84.9069) (size 0.8) (drill 0.4) (layers "F.Cu" "B.Cu") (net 1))
 (segment (start 91.1781 92.6) (end 82.793 92.6) (width 0.25) (layer "B.Cu") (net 1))
 (segment (start 82.793 92.6) (end 76.1688 85.9758) (width 0.25) (layer "B.Cu") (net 1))
 (segment (start 94.3281 95.75) (end 91.1781 92.6) (width 0.25) (layer "B.Cu") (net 1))
 (segment (start 95.955 95.75) (end 94.3281 95.75) (width 0.25) (layer "B.Cu") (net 1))
 (segment (start 76.1688 85.9758) (end 76.1688 84.9069) (width 0.25) (layer "B.Cu") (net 1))
 (segment (start 109.5369 76.1749) (end 109.5369 70.5199) (width 0.25) (layer "F.Cu") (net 4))
 (segment (start 73.2775 90.3467) (end 74.8732 88.751) (width 0.25) (layer "F.Cu") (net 4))
 (segment (start 107.91 65.45) (end 106.1885 67.1715) (width 0.25) (layer "F.Cu") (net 4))
 (segment (start 103.96 69.4) (end 89.15 69.4) (width 0.25) (layer "F.Cu") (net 4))
 (segment (start 106.1885 67.1715) (end 103.96 69.4) (width 0.25) (layer "F.Cu") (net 4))
 (segment (start 73.2775 91.6543) (end 73.2775 90.3467) (width 0.25) (layer "F.Cu") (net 4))
 (segment (start 109.5369 70.5199) (end 106.1885 67.1715) (width 0.25) (layer "F.Cu") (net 4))
 (segment (start 84.5368 79.7867) (end 105.9251 79.7867) (width 0.25) (layer "F.Cu") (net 4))
 (segment (start 82.5433 84.31) (end 82.5433 81.7802) (width 0.25) (layer "F.Cu") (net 4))
 (segment (start 82.5433 81.7802) (end 84.5368 79.7867) (width 0.25) (layer "F.Cu") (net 4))
 (segment (start 105.9251 79.7867) (end 109.5369 76.1749) (width 0.25) (layer "F.Cu") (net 4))
 (segment (start 74.8732 88.751) (end 78.1023 88.751) (width 0.25) (layer "F.Cu") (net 4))
 (segment (start 78.1023 88.751) (end 82.5433 84.31) (width 0.25) (layer "F.Cu") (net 4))
 (segment (start 106.5331 76.8769) (end 89.3769 76.8769) (width 0.25) (layer "F.Cu") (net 7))
 (segment (start 75.8175 92.7812) (end 80.1704 92.7812) (width 0.25) (layer "F.Cu") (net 7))
 (segment (start 80.1704 92.7812) (end 82.1212 90.8304) (width 0.25) (layer "F.Cu") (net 7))
 (segment (start 75.8175 91.6543) (end 75.8175 92.7812) (width 0.25) (layer "F.Cu") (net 7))
 (segment (start 107.91 75.5) (end 106.5331 76.8769) (width 0.25) (layer "F.Cu") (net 7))
 (segment (start 89.3769 76.8769) (end 88.9 76.4) (width 0.25) (layer "F.Cu") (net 7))
 (via (at 82.1212 90.8304) (size 0.8) (drill 0.4) (layers "F.Cu" "B.Cu") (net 7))
 (segment (start 104.3749 79.0351) (end 93.9165 79.0351) (width 0.25) (layer "B.Cu") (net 7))
 (segment (start 107.91 75.5) (end 104.3749 79.0351) (width 0.25) (layer "B.Cu") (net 7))
 (segment (start 93.9165 79.0351) (end 82.1212 90.8304) (width 0.25) (layer "B.Cu") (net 7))
 (segment (start 91.279 83.8318) (end 89.9736 82.5264) (width 0.25) (layer "F.Cu") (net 5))
 (segment (start 89.9736 82.5264) (end 88.9 83.6) (width 0.25) (layer "F.Cu") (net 5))
 (segment (start 89.9736 80.9821) (end 89.9736 82.5264) (width 0.25) (layer "F.Cu") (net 5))
 (segment (start 73.9125 90.3508) (end 74.983 89.2803) (width 0.25) (layer "F.Cu") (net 5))
 (segment (start 83.2032 81.7616) (end 84.3636 80.6012) (width 0.25) (layer "F.Cu") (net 5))
 (segment (start 84.3636 80.6012) (end 89.5927 80.6012) (width 0.25) (layer "F.Cu") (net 5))
 (segment (start 106.2918 83.8318) (end 91.279 83.8318) (width 0.25) (layer "F.Cu") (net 5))
 (segment (start 89.5927 80.6012) (end 89.9736 80.9821) (width 0.25) (layer "F.Cu") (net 5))
 (segment (start 78.2121 89.2803) (end 83.2032 84.2892) (width 0.25) (layer "F.Cu") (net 5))
 (segment (start 74.983 89.2803) (end 78.2121 89.2803) (width 0.25) (layer "F.Cu") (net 5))
 (segment (start 107.91 85.45) (end 106.2918 83.8318) (width 0.25) (layer "F.Cu") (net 5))
 (segment (start 83.2032 84.2892) (end 83.2032 81.7616) (width 0.25) (layer "F.Cu") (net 5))
 (segment (start 73.9125 91.6543) (end 73.9125 90.3508) (width 0.25) (layer "F.Cu") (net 5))
 (segment (start 75.1825 91.6543) (end 75.1825 92.8115) (width 0.25) (layer "F.Cu") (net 3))
 (segment (start 88.6 91.1) (end 91.5624 94.0624) (width 0.25) (layer "F.Cu") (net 3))
 (segment (start 75.1825 92.8115) (end 75.6102 93.2392) (width 0.25) (layer "F.Cu") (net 3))
 (segment (start 83.5 90.9701) (end 83.5 89.5) (width 0.25) (layer "F.Cu") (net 3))
 (segment (start 87.6513 89.0513) (end 88.6 90) (width 0.25) (layer "F.Cu") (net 3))
 (segment (start 75.6102 93.2392) (end 81.2309 93.2392) (width 0.25) (layer "F.Cu") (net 3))
 (segment (start 88.6 90) (end 88.6 91.1) (width 0.25) (layer "F.Cu") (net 3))
 (segment (start 83.5 89.5) (end 83.9487 89.0513) (width 0.25) (layer "F.Cu") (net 3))
 (segment (start 81.2309 93.2392) (end 83.5 90.9701) (width 0.25) (layer "F.Cu") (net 3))
 (segment (start 83.9487 89.0513) (end 87.6513 89.0513) (width 0.25) (layer "F.Cu") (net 3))
 (segment (start 107.91 95.75) (end 106.2224 94.0624) (width 0.25) (layer "F.Cu") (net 3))
 (segment (start 106.2224 94.0624) (end 91.5624 94.0624) (width 0.25) (layer "F.Cu") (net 3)))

